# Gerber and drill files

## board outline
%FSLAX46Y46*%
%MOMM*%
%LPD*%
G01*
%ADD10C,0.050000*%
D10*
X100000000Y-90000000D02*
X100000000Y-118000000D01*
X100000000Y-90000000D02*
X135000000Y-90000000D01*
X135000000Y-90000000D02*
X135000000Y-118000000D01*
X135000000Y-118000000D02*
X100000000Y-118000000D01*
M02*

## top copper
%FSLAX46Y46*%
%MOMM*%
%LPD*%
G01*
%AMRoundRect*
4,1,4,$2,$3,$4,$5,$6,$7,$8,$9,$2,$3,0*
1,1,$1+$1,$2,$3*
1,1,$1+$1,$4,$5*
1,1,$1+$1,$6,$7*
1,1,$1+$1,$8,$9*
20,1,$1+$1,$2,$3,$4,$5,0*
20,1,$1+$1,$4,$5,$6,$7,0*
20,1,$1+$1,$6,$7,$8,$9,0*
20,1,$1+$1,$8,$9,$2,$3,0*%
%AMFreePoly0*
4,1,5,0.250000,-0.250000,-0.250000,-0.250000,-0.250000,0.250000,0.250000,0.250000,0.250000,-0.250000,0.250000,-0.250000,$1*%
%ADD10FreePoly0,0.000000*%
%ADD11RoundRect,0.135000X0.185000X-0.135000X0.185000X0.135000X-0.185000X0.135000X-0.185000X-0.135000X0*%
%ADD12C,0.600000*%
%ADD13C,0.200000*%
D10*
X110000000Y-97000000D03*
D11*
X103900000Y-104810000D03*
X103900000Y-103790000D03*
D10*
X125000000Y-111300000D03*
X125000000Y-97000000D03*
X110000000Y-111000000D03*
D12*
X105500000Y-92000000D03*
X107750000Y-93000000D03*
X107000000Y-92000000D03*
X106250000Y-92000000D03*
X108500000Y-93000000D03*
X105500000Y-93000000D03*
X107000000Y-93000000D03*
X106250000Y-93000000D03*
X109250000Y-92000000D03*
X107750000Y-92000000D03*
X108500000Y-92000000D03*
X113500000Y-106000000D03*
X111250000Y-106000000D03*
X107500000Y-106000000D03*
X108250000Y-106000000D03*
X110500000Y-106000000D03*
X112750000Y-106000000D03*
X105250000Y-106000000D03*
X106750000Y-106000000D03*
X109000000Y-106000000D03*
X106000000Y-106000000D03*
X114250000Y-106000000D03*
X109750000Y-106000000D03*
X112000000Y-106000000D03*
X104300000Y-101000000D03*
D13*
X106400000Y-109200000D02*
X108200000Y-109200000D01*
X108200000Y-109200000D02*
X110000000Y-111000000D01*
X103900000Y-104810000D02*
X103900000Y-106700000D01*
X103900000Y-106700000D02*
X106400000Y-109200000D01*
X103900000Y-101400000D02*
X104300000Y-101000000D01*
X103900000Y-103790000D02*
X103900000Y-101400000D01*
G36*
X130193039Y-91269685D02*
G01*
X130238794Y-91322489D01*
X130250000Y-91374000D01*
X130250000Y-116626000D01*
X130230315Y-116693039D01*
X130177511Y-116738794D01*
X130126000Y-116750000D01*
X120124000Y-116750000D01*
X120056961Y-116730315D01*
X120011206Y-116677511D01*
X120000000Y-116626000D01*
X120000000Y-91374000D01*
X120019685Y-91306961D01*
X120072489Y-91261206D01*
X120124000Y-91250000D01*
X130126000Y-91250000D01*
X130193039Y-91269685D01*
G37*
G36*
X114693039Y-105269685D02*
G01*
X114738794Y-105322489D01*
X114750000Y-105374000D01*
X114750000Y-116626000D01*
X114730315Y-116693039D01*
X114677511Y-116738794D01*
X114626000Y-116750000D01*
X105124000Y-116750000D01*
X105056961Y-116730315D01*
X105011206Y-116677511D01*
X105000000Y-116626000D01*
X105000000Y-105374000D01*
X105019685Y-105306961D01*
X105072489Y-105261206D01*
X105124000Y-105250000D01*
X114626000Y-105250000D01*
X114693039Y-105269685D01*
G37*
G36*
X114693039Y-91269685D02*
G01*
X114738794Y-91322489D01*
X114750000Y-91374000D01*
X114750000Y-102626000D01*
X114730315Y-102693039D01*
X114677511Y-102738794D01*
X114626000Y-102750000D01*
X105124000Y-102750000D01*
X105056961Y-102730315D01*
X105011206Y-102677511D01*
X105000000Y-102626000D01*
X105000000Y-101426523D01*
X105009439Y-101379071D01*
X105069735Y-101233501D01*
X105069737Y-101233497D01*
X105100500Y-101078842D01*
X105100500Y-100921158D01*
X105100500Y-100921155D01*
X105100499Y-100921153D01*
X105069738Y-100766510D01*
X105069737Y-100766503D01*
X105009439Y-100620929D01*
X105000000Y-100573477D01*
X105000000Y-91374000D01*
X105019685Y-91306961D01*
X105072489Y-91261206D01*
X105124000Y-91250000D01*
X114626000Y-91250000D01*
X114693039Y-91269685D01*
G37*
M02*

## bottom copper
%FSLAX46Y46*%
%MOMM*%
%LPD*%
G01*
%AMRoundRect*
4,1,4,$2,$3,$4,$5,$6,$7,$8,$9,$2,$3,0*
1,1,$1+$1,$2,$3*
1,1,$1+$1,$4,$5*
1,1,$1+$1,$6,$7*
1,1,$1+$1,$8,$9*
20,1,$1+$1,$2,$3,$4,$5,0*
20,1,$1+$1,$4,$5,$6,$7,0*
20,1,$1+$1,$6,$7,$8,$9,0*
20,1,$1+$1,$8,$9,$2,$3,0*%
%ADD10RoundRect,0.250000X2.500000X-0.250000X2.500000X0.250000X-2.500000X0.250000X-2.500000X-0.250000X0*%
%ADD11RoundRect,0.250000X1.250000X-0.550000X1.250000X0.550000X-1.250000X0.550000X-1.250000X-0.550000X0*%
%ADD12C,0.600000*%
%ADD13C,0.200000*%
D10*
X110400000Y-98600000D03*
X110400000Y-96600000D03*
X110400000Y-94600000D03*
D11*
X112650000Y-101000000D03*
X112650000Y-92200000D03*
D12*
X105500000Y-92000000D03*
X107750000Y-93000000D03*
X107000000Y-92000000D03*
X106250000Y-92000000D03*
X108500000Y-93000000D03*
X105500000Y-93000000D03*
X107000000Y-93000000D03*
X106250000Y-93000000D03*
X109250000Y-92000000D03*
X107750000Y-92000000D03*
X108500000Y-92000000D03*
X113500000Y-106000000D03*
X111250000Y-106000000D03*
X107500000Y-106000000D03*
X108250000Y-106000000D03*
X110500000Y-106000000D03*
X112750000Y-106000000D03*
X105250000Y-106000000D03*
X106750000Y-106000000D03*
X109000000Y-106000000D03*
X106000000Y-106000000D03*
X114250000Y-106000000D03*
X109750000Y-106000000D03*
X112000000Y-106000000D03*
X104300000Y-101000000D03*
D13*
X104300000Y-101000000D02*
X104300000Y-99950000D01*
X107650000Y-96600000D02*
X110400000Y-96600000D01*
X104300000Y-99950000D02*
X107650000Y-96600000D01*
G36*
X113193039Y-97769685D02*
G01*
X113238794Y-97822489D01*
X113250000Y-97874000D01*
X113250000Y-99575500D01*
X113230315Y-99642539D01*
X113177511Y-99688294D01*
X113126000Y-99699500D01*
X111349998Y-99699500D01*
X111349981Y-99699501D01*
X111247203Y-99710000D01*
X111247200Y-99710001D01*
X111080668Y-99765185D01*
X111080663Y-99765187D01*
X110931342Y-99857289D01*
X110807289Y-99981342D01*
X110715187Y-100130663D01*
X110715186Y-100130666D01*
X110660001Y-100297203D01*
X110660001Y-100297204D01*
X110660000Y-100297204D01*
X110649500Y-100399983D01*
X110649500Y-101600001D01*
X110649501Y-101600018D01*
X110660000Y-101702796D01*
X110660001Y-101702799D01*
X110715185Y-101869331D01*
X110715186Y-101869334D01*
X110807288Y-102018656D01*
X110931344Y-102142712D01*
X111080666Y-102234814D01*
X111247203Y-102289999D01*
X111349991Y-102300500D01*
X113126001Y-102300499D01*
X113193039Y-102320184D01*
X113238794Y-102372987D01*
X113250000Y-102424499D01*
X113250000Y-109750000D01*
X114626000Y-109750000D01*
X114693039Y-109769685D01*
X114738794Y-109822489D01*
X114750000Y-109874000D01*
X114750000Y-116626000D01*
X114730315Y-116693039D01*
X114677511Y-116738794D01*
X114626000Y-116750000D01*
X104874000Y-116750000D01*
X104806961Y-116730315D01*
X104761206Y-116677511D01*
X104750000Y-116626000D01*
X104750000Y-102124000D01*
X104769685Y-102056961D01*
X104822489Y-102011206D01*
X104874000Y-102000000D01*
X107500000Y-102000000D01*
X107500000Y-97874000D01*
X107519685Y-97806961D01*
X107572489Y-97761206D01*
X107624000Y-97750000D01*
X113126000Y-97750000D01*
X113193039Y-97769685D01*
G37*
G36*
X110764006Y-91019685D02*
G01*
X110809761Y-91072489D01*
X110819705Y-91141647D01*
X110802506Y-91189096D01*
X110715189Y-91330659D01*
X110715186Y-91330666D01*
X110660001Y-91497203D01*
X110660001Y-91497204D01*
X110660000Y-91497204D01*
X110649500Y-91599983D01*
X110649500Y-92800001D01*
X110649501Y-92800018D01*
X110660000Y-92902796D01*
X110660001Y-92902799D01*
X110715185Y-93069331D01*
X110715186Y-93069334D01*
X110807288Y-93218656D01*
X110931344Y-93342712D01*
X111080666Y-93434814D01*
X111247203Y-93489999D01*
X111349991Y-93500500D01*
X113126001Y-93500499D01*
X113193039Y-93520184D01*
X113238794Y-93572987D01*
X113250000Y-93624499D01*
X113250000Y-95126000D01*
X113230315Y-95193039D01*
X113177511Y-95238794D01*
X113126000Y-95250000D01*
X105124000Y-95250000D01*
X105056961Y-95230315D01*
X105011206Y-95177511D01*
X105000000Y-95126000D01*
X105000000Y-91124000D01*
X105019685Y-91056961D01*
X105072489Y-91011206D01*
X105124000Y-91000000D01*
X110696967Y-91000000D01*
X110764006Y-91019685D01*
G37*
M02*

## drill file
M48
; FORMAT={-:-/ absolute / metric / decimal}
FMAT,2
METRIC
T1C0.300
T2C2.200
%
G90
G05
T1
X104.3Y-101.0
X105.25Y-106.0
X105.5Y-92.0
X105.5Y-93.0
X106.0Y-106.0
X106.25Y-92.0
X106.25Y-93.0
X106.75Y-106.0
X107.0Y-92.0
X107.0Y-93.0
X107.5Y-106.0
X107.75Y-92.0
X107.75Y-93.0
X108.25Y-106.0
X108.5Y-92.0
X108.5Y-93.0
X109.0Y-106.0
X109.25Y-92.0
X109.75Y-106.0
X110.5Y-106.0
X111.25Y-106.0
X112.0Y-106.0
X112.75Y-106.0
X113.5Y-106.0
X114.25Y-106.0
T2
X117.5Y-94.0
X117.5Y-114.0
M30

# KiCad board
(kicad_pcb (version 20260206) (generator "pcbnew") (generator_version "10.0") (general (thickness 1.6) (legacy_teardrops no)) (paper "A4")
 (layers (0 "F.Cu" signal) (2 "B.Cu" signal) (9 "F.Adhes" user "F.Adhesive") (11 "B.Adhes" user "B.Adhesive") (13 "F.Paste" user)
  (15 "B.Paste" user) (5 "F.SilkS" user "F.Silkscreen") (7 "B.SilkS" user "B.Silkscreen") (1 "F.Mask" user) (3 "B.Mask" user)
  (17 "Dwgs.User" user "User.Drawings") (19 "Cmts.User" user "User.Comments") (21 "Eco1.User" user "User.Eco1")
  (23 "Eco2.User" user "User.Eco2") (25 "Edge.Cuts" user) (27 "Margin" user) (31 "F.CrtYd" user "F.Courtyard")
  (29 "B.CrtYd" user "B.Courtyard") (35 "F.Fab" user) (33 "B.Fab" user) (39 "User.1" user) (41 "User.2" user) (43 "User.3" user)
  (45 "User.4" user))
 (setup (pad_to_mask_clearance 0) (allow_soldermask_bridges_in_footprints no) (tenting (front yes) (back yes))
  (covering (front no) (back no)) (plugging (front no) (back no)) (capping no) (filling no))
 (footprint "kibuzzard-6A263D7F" (layer "F.Cu") (at 102.5 115.75)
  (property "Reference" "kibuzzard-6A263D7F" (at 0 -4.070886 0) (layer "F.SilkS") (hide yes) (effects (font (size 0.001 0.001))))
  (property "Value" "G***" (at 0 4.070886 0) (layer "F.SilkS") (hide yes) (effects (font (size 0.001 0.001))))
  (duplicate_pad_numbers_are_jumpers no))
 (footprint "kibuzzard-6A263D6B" (layer "F.Cu") (at 102.5 92.5)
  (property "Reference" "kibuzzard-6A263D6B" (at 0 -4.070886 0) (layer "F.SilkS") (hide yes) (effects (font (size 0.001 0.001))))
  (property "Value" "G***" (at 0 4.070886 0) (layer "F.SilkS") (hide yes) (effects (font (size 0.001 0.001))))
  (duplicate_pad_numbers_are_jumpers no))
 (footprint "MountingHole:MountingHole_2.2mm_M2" (layer "F.Cu") (at 117.5 94)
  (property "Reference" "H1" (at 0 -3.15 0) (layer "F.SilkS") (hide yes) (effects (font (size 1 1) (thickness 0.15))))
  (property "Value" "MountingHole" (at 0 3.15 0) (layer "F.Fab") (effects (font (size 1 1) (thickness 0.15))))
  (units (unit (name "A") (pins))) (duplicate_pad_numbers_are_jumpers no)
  (pad "" np_thru_hole circle (at 0 0) (size 2.2 2.2) (drill 2.2) (layers "*.Cu" "*.Mask")))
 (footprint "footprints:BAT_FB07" (layer "F.Cu") (at 110 97)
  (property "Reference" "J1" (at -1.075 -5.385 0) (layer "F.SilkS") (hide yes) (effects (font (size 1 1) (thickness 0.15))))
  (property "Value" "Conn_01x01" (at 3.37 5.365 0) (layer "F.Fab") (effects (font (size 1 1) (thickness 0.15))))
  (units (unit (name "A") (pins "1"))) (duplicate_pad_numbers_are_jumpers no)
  (pad "1" smd custom (at 0 0) (size 0.5 0.5) (layers "F.Cu") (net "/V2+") (options (clearance outline) (anchor rect)) (primitives)))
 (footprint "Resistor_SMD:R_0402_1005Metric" (layer "F.Cu") (at 103.9 104.3 90)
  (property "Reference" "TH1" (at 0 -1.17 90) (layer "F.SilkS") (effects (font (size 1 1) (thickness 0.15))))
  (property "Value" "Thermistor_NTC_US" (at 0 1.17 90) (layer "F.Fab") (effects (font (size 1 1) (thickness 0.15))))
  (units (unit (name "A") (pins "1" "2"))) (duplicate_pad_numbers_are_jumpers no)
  (pad "1" smd roundrect (at -0.51 0 90) (size 0.54 0.64) (layers "F.Cu" "F.Mask" "F.Paste") (roundrect_rratio 0.25) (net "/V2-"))
  (pad "2" smd roundrect (at 0.51 0 90) (size 0.54 0.64) (layers "F.Cu" "F.Mask" "F.Paste") (roundrect_rratio 0.25) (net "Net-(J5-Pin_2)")))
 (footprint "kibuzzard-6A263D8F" (layer "F.Cu") (at 132.5 92.25)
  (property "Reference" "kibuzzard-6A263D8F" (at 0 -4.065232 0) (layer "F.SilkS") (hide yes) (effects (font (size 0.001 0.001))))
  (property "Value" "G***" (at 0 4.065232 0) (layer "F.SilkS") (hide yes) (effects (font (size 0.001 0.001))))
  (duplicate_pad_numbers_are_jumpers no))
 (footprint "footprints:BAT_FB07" (layer "F.Cu") (at 125 111.3)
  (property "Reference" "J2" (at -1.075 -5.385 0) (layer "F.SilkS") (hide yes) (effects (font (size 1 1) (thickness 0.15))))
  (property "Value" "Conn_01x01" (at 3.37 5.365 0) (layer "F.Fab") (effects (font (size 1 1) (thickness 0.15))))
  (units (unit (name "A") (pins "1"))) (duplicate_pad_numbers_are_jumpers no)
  (pad "1" smd custom (at 0 0) (size 0.5 0.5) (layers "F.Cu") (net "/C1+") (options (clearance outline) (anchor rect)) (primitives)))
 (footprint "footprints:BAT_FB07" (layer "F.Cu") (at 125 97)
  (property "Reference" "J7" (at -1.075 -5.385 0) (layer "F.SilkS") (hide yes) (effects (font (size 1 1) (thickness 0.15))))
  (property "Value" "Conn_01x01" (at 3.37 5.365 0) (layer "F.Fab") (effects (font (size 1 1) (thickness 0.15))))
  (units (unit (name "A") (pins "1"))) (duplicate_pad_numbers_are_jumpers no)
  (pad "1" smd custom (at 0 0) (size 0.5 0.5) (layers "F.Cu") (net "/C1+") (options (clearance outline) (anchor rect)) (primitives)))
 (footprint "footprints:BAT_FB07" (layer "F.Cu") (at 110 111)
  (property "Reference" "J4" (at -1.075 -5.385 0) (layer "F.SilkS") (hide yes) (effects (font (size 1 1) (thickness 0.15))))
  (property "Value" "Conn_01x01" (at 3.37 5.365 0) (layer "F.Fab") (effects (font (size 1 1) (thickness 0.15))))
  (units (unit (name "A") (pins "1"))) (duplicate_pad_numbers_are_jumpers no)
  (pad "1" smd custom (at 0 0) (size 0.5 0.5) (layers "F.Cu") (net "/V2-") (options (clearance outline) (anchor rect)) (primitives)))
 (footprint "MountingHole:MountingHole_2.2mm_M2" (layer "F.Cu") (at 117.5 114)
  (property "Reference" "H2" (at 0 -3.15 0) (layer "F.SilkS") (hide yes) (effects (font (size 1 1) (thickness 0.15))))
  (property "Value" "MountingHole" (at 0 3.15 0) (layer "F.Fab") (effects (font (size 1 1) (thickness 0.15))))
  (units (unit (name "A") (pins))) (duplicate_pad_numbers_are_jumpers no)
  (pad "" np_thru_hole circle (at 0 0) (size 2.2 2.2) (drill 2.2) (layers "*.Cu" "*.Mask")))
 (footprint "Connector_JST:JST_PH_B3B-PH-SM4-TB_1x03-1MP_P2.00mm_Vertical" (layer "B.Cu") (at 110.9 96.6 90)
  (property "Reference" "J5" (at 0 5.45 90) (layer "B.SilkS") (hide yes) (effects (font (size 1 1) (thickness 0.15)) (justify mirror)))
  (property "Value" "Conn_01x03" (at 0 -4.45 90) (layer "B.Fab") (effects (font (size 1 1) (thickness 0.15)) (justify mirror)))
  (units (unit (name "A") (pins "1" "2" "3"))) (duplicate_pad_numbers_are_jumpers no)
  (pad "1" smd roundrect (at -2 -0.5 90) (size 1 5.5) (layers "B.Cu" "B.Mask" "B.Paste") (roundrect_rratio 0.25) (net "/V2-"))
  (pad "2" smd roundrect (at 0 -0.5 90) (size 1 5.5) (layers "B.Cu" "B.Mask" "B.Paste") (roundrect_rratio 0.25) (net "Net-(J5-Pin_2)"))
  (pad "3" smd roundrect (at 2 -0.5 90) (size 1 5.5) (layers "B.Cu" "B.Mask" "B.Paste") (roundrect_rratio 0.25) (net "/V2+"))
  (pad "MP" smd roundrect (at -4.4 1.75 90) (size 1.6 3) (layers "B.Cu" "B.Mask" "B.Paste") (roundrect_rratio 0.15625))
  (pad "MP" smd roundrect (at 4.4 1.75 90) (size 1.6 3) (layers "B.Cu" "B.Mask" "B.Paste") (roundrect_rratio 0.15625)))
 (gr_line (start 100 90) (end 100 118) (stroke (width 0.05) (type default)) (layer "Edge.Cuts"))
 (gr_line (start 100 90) (end 135 90) (stroke (width 0.05) (type default)) (layer "Edge.Cuts"))
 (gr_line (start 135 90) (end 135 118) (stroke (width 0.05) (type default)) (layer "Edge.Cuts"))
 (gr_line (start 135 118) (end 100 118) (stroke (width 0.05) (type default)) (layer "Edge.Cuts"))
 (via (at 105.5 92) (size 0.6) (drill 0.3) (layers "F.Cu" "B.Cu") (free yes) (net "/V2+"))
 (via (at 107.75 93) (size 0.6) (drill 0.3) (layers "F.Cu" "B.Cu") (free yes) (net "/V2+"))
 (via (at 107 92) (size 0.6) (drill 0.3) (layers "F.Cu" "B.Cu") (free yes) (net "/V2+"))
 (via (at 106.25 92) (size 0.6) (drill 0.3) (layers "F.Cu" "B.Cu") (free yes) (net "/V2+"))
 (via (at 108.5 93) (size 0.6) (drill 0.3) (layers "F.Cu" "B.Cu") (free yes) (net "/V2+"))
 (via (at 105.5 93) (size 0.6) (drill 0.3) (layers "F.Cu" "B.Cu") (free yes) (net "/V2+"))
 (via (at 107 93) (size 0.6) (drill 0.3) (layers "F.Cu" "B.Cu") (free yes) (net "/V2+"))
 (via (at 106.25 93) (size 0.6) (drill 0.3) (layers "F.Cu" "B.Cu") (free yes) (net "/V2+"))
 (via (at 109.25 92) (size 0.6) (drill 0.3) (layers "F.Cu" "B.Cu") (free yes) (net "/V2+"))
 (via (at 107.75 92) (size 0.6) (drill 0.3) (layers "F.Cu" "B.Cu") (free yes) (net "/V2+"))
 (via (at 108.5 92) (size 0.6) (drill 0.3) (layers "F.Cu" "B.Cu") (free yes) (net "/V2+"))
 (segment (start 106.4 109.2) (end 108.2 109.2) (width 0.2) (layer "F.Cu") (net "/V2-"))
 (segment (start 108.2 109.2) (end 110 111) (width 0.2) (layer "F.Cu") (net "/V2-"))
 (segment (start 103.9 104.81) (end 103.9 106.7) (width 0.2) (layer "F.Cu") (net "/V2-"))
 (segment (start 103.9 106.7) (end 106.4 109.2) (width 0.2) (layer "F.Cu") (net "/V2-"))
 (via (at 113.5 106) (size 0.6) (drill 0.3) (layers "F.Cu" "B.Cu") (free yes) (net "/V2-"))
 (via (at 111.25 106) (size 0.6) (drill 0.3) (layers "F.Cu" "B.Cu") (free yes) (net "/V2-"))
 (via (at 107.5 106) (size 0.6) (drill 0.3) (layers "F.Cu" "B.Cu") (free yes) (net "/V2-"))
 (via (at 108.25 106) (size 0.6) (drill 0.3) (layers "F.Cu" "B.Cu") (free yes) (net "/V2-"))
 (via (at 110.5 106) (size 0.6) (drill 0.3) (layers "F.Cu" "B.Cu") (free yes) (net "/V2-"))
 (via (at 112.75 106) (size 0.6) (drill 0.3) (layers "F.Cu" "B.Cu") (free yes) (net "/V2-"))
 (via (at 105.25 106) (size 0.6) (drill 0.3) (layers "F.Cu" "B.Cu") (free yes) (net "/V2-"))
 (via (at 106.75 106) (size 0.6) (drill 0.3) (layers "F.Cu" "B.Cu") (free yes) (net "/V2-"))
 (via (at 109 106) (size 0.6) (drill 0.3) (layers "F.Cu" "B.Cu") (free yes) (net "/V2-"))
 (via (at 106 106) (size 0.6) (drill 0.3) (layers "F.Cu" "B.Cu") (free yes) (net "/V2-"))
 (via (at 114.25 106) (size 0.6) (drill 0.3) (layers "F.Cu" "B.Cu") (free yes) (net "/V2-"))
 (via (at 109.75 106) (size 0.6) (drill 0.3) (layers "F.Cu" "B.Cu") (free yes) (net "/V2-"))
 (via (at 112 106) (size 0.6) (drill 0.3) (layers "F.Cu" "B.Cu") (free yes) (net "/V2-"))
 (segment (start 103.9 101.4) (end 104.3 101) (width 0.2) (layer "F.Cu") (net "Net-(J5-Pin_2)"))
 (segment (start 103.9 103.79) (end 103.9 101.4) (width 0.2) (layer "F.Cu") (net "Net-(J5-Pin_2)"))
 (via (at 104.3 101) (size 0.6) (drill 0.3) (layers "F.Cu" "B.Cu") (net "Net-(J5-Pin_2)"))
 (segment (start 104.3 101) (end 104.3 99.95) (width 0.2) (layer "B.Cu") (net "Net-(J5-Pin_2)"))
 (segment (start 107.65 96.6) (end 110.4 96.6) (width 0.2) (layer "B.Cu") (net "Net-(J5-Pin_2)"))
 (segment (start 104.3 99.95) (end 107.65 96.6) (width 0.2) (layer "B.Cu") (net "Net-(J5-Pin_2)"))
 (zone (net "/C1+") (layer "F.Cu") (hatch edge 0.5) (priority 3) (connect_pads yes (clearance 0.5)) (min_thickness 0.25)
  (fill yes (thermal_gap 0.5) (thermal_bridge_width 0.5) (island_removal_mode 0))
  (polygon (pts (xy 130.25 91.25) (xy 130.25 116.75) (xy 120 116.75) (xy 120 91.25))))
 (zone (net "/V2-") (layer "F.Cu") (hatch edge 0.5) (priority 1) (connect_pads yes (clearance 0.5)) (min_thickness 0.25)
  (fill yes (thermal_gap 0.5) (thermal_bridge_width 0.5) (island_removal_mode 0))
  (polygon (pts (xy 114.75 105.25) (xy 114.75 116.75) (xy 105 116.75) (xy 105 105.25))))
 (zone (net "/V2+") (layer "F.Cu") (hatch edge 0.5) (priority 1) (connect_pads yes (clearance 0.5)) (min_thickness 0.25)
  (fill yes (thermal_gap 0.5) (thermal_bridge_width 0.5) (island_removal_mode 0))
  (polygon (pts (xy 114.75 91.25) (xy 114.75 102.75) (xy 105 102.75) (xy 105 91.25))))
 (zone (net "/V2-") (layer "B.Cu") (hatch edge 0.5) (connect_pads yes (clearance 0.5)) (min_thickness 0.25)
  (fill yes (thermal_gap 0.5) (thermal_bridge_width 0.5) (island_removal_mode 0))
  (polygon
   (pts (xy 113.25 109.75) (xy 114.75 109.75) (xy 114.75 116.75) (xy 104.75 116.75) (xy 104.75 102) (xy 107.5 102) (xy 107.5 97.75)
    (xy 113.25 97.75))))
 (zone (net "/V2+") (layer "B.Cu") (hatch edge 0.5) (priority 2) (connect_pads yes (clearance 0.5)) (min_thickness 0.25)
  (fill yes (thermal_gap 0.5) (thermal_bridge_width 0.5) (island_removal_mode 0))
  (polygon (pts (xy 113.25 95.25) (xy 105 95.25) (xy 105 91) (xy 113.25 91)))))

